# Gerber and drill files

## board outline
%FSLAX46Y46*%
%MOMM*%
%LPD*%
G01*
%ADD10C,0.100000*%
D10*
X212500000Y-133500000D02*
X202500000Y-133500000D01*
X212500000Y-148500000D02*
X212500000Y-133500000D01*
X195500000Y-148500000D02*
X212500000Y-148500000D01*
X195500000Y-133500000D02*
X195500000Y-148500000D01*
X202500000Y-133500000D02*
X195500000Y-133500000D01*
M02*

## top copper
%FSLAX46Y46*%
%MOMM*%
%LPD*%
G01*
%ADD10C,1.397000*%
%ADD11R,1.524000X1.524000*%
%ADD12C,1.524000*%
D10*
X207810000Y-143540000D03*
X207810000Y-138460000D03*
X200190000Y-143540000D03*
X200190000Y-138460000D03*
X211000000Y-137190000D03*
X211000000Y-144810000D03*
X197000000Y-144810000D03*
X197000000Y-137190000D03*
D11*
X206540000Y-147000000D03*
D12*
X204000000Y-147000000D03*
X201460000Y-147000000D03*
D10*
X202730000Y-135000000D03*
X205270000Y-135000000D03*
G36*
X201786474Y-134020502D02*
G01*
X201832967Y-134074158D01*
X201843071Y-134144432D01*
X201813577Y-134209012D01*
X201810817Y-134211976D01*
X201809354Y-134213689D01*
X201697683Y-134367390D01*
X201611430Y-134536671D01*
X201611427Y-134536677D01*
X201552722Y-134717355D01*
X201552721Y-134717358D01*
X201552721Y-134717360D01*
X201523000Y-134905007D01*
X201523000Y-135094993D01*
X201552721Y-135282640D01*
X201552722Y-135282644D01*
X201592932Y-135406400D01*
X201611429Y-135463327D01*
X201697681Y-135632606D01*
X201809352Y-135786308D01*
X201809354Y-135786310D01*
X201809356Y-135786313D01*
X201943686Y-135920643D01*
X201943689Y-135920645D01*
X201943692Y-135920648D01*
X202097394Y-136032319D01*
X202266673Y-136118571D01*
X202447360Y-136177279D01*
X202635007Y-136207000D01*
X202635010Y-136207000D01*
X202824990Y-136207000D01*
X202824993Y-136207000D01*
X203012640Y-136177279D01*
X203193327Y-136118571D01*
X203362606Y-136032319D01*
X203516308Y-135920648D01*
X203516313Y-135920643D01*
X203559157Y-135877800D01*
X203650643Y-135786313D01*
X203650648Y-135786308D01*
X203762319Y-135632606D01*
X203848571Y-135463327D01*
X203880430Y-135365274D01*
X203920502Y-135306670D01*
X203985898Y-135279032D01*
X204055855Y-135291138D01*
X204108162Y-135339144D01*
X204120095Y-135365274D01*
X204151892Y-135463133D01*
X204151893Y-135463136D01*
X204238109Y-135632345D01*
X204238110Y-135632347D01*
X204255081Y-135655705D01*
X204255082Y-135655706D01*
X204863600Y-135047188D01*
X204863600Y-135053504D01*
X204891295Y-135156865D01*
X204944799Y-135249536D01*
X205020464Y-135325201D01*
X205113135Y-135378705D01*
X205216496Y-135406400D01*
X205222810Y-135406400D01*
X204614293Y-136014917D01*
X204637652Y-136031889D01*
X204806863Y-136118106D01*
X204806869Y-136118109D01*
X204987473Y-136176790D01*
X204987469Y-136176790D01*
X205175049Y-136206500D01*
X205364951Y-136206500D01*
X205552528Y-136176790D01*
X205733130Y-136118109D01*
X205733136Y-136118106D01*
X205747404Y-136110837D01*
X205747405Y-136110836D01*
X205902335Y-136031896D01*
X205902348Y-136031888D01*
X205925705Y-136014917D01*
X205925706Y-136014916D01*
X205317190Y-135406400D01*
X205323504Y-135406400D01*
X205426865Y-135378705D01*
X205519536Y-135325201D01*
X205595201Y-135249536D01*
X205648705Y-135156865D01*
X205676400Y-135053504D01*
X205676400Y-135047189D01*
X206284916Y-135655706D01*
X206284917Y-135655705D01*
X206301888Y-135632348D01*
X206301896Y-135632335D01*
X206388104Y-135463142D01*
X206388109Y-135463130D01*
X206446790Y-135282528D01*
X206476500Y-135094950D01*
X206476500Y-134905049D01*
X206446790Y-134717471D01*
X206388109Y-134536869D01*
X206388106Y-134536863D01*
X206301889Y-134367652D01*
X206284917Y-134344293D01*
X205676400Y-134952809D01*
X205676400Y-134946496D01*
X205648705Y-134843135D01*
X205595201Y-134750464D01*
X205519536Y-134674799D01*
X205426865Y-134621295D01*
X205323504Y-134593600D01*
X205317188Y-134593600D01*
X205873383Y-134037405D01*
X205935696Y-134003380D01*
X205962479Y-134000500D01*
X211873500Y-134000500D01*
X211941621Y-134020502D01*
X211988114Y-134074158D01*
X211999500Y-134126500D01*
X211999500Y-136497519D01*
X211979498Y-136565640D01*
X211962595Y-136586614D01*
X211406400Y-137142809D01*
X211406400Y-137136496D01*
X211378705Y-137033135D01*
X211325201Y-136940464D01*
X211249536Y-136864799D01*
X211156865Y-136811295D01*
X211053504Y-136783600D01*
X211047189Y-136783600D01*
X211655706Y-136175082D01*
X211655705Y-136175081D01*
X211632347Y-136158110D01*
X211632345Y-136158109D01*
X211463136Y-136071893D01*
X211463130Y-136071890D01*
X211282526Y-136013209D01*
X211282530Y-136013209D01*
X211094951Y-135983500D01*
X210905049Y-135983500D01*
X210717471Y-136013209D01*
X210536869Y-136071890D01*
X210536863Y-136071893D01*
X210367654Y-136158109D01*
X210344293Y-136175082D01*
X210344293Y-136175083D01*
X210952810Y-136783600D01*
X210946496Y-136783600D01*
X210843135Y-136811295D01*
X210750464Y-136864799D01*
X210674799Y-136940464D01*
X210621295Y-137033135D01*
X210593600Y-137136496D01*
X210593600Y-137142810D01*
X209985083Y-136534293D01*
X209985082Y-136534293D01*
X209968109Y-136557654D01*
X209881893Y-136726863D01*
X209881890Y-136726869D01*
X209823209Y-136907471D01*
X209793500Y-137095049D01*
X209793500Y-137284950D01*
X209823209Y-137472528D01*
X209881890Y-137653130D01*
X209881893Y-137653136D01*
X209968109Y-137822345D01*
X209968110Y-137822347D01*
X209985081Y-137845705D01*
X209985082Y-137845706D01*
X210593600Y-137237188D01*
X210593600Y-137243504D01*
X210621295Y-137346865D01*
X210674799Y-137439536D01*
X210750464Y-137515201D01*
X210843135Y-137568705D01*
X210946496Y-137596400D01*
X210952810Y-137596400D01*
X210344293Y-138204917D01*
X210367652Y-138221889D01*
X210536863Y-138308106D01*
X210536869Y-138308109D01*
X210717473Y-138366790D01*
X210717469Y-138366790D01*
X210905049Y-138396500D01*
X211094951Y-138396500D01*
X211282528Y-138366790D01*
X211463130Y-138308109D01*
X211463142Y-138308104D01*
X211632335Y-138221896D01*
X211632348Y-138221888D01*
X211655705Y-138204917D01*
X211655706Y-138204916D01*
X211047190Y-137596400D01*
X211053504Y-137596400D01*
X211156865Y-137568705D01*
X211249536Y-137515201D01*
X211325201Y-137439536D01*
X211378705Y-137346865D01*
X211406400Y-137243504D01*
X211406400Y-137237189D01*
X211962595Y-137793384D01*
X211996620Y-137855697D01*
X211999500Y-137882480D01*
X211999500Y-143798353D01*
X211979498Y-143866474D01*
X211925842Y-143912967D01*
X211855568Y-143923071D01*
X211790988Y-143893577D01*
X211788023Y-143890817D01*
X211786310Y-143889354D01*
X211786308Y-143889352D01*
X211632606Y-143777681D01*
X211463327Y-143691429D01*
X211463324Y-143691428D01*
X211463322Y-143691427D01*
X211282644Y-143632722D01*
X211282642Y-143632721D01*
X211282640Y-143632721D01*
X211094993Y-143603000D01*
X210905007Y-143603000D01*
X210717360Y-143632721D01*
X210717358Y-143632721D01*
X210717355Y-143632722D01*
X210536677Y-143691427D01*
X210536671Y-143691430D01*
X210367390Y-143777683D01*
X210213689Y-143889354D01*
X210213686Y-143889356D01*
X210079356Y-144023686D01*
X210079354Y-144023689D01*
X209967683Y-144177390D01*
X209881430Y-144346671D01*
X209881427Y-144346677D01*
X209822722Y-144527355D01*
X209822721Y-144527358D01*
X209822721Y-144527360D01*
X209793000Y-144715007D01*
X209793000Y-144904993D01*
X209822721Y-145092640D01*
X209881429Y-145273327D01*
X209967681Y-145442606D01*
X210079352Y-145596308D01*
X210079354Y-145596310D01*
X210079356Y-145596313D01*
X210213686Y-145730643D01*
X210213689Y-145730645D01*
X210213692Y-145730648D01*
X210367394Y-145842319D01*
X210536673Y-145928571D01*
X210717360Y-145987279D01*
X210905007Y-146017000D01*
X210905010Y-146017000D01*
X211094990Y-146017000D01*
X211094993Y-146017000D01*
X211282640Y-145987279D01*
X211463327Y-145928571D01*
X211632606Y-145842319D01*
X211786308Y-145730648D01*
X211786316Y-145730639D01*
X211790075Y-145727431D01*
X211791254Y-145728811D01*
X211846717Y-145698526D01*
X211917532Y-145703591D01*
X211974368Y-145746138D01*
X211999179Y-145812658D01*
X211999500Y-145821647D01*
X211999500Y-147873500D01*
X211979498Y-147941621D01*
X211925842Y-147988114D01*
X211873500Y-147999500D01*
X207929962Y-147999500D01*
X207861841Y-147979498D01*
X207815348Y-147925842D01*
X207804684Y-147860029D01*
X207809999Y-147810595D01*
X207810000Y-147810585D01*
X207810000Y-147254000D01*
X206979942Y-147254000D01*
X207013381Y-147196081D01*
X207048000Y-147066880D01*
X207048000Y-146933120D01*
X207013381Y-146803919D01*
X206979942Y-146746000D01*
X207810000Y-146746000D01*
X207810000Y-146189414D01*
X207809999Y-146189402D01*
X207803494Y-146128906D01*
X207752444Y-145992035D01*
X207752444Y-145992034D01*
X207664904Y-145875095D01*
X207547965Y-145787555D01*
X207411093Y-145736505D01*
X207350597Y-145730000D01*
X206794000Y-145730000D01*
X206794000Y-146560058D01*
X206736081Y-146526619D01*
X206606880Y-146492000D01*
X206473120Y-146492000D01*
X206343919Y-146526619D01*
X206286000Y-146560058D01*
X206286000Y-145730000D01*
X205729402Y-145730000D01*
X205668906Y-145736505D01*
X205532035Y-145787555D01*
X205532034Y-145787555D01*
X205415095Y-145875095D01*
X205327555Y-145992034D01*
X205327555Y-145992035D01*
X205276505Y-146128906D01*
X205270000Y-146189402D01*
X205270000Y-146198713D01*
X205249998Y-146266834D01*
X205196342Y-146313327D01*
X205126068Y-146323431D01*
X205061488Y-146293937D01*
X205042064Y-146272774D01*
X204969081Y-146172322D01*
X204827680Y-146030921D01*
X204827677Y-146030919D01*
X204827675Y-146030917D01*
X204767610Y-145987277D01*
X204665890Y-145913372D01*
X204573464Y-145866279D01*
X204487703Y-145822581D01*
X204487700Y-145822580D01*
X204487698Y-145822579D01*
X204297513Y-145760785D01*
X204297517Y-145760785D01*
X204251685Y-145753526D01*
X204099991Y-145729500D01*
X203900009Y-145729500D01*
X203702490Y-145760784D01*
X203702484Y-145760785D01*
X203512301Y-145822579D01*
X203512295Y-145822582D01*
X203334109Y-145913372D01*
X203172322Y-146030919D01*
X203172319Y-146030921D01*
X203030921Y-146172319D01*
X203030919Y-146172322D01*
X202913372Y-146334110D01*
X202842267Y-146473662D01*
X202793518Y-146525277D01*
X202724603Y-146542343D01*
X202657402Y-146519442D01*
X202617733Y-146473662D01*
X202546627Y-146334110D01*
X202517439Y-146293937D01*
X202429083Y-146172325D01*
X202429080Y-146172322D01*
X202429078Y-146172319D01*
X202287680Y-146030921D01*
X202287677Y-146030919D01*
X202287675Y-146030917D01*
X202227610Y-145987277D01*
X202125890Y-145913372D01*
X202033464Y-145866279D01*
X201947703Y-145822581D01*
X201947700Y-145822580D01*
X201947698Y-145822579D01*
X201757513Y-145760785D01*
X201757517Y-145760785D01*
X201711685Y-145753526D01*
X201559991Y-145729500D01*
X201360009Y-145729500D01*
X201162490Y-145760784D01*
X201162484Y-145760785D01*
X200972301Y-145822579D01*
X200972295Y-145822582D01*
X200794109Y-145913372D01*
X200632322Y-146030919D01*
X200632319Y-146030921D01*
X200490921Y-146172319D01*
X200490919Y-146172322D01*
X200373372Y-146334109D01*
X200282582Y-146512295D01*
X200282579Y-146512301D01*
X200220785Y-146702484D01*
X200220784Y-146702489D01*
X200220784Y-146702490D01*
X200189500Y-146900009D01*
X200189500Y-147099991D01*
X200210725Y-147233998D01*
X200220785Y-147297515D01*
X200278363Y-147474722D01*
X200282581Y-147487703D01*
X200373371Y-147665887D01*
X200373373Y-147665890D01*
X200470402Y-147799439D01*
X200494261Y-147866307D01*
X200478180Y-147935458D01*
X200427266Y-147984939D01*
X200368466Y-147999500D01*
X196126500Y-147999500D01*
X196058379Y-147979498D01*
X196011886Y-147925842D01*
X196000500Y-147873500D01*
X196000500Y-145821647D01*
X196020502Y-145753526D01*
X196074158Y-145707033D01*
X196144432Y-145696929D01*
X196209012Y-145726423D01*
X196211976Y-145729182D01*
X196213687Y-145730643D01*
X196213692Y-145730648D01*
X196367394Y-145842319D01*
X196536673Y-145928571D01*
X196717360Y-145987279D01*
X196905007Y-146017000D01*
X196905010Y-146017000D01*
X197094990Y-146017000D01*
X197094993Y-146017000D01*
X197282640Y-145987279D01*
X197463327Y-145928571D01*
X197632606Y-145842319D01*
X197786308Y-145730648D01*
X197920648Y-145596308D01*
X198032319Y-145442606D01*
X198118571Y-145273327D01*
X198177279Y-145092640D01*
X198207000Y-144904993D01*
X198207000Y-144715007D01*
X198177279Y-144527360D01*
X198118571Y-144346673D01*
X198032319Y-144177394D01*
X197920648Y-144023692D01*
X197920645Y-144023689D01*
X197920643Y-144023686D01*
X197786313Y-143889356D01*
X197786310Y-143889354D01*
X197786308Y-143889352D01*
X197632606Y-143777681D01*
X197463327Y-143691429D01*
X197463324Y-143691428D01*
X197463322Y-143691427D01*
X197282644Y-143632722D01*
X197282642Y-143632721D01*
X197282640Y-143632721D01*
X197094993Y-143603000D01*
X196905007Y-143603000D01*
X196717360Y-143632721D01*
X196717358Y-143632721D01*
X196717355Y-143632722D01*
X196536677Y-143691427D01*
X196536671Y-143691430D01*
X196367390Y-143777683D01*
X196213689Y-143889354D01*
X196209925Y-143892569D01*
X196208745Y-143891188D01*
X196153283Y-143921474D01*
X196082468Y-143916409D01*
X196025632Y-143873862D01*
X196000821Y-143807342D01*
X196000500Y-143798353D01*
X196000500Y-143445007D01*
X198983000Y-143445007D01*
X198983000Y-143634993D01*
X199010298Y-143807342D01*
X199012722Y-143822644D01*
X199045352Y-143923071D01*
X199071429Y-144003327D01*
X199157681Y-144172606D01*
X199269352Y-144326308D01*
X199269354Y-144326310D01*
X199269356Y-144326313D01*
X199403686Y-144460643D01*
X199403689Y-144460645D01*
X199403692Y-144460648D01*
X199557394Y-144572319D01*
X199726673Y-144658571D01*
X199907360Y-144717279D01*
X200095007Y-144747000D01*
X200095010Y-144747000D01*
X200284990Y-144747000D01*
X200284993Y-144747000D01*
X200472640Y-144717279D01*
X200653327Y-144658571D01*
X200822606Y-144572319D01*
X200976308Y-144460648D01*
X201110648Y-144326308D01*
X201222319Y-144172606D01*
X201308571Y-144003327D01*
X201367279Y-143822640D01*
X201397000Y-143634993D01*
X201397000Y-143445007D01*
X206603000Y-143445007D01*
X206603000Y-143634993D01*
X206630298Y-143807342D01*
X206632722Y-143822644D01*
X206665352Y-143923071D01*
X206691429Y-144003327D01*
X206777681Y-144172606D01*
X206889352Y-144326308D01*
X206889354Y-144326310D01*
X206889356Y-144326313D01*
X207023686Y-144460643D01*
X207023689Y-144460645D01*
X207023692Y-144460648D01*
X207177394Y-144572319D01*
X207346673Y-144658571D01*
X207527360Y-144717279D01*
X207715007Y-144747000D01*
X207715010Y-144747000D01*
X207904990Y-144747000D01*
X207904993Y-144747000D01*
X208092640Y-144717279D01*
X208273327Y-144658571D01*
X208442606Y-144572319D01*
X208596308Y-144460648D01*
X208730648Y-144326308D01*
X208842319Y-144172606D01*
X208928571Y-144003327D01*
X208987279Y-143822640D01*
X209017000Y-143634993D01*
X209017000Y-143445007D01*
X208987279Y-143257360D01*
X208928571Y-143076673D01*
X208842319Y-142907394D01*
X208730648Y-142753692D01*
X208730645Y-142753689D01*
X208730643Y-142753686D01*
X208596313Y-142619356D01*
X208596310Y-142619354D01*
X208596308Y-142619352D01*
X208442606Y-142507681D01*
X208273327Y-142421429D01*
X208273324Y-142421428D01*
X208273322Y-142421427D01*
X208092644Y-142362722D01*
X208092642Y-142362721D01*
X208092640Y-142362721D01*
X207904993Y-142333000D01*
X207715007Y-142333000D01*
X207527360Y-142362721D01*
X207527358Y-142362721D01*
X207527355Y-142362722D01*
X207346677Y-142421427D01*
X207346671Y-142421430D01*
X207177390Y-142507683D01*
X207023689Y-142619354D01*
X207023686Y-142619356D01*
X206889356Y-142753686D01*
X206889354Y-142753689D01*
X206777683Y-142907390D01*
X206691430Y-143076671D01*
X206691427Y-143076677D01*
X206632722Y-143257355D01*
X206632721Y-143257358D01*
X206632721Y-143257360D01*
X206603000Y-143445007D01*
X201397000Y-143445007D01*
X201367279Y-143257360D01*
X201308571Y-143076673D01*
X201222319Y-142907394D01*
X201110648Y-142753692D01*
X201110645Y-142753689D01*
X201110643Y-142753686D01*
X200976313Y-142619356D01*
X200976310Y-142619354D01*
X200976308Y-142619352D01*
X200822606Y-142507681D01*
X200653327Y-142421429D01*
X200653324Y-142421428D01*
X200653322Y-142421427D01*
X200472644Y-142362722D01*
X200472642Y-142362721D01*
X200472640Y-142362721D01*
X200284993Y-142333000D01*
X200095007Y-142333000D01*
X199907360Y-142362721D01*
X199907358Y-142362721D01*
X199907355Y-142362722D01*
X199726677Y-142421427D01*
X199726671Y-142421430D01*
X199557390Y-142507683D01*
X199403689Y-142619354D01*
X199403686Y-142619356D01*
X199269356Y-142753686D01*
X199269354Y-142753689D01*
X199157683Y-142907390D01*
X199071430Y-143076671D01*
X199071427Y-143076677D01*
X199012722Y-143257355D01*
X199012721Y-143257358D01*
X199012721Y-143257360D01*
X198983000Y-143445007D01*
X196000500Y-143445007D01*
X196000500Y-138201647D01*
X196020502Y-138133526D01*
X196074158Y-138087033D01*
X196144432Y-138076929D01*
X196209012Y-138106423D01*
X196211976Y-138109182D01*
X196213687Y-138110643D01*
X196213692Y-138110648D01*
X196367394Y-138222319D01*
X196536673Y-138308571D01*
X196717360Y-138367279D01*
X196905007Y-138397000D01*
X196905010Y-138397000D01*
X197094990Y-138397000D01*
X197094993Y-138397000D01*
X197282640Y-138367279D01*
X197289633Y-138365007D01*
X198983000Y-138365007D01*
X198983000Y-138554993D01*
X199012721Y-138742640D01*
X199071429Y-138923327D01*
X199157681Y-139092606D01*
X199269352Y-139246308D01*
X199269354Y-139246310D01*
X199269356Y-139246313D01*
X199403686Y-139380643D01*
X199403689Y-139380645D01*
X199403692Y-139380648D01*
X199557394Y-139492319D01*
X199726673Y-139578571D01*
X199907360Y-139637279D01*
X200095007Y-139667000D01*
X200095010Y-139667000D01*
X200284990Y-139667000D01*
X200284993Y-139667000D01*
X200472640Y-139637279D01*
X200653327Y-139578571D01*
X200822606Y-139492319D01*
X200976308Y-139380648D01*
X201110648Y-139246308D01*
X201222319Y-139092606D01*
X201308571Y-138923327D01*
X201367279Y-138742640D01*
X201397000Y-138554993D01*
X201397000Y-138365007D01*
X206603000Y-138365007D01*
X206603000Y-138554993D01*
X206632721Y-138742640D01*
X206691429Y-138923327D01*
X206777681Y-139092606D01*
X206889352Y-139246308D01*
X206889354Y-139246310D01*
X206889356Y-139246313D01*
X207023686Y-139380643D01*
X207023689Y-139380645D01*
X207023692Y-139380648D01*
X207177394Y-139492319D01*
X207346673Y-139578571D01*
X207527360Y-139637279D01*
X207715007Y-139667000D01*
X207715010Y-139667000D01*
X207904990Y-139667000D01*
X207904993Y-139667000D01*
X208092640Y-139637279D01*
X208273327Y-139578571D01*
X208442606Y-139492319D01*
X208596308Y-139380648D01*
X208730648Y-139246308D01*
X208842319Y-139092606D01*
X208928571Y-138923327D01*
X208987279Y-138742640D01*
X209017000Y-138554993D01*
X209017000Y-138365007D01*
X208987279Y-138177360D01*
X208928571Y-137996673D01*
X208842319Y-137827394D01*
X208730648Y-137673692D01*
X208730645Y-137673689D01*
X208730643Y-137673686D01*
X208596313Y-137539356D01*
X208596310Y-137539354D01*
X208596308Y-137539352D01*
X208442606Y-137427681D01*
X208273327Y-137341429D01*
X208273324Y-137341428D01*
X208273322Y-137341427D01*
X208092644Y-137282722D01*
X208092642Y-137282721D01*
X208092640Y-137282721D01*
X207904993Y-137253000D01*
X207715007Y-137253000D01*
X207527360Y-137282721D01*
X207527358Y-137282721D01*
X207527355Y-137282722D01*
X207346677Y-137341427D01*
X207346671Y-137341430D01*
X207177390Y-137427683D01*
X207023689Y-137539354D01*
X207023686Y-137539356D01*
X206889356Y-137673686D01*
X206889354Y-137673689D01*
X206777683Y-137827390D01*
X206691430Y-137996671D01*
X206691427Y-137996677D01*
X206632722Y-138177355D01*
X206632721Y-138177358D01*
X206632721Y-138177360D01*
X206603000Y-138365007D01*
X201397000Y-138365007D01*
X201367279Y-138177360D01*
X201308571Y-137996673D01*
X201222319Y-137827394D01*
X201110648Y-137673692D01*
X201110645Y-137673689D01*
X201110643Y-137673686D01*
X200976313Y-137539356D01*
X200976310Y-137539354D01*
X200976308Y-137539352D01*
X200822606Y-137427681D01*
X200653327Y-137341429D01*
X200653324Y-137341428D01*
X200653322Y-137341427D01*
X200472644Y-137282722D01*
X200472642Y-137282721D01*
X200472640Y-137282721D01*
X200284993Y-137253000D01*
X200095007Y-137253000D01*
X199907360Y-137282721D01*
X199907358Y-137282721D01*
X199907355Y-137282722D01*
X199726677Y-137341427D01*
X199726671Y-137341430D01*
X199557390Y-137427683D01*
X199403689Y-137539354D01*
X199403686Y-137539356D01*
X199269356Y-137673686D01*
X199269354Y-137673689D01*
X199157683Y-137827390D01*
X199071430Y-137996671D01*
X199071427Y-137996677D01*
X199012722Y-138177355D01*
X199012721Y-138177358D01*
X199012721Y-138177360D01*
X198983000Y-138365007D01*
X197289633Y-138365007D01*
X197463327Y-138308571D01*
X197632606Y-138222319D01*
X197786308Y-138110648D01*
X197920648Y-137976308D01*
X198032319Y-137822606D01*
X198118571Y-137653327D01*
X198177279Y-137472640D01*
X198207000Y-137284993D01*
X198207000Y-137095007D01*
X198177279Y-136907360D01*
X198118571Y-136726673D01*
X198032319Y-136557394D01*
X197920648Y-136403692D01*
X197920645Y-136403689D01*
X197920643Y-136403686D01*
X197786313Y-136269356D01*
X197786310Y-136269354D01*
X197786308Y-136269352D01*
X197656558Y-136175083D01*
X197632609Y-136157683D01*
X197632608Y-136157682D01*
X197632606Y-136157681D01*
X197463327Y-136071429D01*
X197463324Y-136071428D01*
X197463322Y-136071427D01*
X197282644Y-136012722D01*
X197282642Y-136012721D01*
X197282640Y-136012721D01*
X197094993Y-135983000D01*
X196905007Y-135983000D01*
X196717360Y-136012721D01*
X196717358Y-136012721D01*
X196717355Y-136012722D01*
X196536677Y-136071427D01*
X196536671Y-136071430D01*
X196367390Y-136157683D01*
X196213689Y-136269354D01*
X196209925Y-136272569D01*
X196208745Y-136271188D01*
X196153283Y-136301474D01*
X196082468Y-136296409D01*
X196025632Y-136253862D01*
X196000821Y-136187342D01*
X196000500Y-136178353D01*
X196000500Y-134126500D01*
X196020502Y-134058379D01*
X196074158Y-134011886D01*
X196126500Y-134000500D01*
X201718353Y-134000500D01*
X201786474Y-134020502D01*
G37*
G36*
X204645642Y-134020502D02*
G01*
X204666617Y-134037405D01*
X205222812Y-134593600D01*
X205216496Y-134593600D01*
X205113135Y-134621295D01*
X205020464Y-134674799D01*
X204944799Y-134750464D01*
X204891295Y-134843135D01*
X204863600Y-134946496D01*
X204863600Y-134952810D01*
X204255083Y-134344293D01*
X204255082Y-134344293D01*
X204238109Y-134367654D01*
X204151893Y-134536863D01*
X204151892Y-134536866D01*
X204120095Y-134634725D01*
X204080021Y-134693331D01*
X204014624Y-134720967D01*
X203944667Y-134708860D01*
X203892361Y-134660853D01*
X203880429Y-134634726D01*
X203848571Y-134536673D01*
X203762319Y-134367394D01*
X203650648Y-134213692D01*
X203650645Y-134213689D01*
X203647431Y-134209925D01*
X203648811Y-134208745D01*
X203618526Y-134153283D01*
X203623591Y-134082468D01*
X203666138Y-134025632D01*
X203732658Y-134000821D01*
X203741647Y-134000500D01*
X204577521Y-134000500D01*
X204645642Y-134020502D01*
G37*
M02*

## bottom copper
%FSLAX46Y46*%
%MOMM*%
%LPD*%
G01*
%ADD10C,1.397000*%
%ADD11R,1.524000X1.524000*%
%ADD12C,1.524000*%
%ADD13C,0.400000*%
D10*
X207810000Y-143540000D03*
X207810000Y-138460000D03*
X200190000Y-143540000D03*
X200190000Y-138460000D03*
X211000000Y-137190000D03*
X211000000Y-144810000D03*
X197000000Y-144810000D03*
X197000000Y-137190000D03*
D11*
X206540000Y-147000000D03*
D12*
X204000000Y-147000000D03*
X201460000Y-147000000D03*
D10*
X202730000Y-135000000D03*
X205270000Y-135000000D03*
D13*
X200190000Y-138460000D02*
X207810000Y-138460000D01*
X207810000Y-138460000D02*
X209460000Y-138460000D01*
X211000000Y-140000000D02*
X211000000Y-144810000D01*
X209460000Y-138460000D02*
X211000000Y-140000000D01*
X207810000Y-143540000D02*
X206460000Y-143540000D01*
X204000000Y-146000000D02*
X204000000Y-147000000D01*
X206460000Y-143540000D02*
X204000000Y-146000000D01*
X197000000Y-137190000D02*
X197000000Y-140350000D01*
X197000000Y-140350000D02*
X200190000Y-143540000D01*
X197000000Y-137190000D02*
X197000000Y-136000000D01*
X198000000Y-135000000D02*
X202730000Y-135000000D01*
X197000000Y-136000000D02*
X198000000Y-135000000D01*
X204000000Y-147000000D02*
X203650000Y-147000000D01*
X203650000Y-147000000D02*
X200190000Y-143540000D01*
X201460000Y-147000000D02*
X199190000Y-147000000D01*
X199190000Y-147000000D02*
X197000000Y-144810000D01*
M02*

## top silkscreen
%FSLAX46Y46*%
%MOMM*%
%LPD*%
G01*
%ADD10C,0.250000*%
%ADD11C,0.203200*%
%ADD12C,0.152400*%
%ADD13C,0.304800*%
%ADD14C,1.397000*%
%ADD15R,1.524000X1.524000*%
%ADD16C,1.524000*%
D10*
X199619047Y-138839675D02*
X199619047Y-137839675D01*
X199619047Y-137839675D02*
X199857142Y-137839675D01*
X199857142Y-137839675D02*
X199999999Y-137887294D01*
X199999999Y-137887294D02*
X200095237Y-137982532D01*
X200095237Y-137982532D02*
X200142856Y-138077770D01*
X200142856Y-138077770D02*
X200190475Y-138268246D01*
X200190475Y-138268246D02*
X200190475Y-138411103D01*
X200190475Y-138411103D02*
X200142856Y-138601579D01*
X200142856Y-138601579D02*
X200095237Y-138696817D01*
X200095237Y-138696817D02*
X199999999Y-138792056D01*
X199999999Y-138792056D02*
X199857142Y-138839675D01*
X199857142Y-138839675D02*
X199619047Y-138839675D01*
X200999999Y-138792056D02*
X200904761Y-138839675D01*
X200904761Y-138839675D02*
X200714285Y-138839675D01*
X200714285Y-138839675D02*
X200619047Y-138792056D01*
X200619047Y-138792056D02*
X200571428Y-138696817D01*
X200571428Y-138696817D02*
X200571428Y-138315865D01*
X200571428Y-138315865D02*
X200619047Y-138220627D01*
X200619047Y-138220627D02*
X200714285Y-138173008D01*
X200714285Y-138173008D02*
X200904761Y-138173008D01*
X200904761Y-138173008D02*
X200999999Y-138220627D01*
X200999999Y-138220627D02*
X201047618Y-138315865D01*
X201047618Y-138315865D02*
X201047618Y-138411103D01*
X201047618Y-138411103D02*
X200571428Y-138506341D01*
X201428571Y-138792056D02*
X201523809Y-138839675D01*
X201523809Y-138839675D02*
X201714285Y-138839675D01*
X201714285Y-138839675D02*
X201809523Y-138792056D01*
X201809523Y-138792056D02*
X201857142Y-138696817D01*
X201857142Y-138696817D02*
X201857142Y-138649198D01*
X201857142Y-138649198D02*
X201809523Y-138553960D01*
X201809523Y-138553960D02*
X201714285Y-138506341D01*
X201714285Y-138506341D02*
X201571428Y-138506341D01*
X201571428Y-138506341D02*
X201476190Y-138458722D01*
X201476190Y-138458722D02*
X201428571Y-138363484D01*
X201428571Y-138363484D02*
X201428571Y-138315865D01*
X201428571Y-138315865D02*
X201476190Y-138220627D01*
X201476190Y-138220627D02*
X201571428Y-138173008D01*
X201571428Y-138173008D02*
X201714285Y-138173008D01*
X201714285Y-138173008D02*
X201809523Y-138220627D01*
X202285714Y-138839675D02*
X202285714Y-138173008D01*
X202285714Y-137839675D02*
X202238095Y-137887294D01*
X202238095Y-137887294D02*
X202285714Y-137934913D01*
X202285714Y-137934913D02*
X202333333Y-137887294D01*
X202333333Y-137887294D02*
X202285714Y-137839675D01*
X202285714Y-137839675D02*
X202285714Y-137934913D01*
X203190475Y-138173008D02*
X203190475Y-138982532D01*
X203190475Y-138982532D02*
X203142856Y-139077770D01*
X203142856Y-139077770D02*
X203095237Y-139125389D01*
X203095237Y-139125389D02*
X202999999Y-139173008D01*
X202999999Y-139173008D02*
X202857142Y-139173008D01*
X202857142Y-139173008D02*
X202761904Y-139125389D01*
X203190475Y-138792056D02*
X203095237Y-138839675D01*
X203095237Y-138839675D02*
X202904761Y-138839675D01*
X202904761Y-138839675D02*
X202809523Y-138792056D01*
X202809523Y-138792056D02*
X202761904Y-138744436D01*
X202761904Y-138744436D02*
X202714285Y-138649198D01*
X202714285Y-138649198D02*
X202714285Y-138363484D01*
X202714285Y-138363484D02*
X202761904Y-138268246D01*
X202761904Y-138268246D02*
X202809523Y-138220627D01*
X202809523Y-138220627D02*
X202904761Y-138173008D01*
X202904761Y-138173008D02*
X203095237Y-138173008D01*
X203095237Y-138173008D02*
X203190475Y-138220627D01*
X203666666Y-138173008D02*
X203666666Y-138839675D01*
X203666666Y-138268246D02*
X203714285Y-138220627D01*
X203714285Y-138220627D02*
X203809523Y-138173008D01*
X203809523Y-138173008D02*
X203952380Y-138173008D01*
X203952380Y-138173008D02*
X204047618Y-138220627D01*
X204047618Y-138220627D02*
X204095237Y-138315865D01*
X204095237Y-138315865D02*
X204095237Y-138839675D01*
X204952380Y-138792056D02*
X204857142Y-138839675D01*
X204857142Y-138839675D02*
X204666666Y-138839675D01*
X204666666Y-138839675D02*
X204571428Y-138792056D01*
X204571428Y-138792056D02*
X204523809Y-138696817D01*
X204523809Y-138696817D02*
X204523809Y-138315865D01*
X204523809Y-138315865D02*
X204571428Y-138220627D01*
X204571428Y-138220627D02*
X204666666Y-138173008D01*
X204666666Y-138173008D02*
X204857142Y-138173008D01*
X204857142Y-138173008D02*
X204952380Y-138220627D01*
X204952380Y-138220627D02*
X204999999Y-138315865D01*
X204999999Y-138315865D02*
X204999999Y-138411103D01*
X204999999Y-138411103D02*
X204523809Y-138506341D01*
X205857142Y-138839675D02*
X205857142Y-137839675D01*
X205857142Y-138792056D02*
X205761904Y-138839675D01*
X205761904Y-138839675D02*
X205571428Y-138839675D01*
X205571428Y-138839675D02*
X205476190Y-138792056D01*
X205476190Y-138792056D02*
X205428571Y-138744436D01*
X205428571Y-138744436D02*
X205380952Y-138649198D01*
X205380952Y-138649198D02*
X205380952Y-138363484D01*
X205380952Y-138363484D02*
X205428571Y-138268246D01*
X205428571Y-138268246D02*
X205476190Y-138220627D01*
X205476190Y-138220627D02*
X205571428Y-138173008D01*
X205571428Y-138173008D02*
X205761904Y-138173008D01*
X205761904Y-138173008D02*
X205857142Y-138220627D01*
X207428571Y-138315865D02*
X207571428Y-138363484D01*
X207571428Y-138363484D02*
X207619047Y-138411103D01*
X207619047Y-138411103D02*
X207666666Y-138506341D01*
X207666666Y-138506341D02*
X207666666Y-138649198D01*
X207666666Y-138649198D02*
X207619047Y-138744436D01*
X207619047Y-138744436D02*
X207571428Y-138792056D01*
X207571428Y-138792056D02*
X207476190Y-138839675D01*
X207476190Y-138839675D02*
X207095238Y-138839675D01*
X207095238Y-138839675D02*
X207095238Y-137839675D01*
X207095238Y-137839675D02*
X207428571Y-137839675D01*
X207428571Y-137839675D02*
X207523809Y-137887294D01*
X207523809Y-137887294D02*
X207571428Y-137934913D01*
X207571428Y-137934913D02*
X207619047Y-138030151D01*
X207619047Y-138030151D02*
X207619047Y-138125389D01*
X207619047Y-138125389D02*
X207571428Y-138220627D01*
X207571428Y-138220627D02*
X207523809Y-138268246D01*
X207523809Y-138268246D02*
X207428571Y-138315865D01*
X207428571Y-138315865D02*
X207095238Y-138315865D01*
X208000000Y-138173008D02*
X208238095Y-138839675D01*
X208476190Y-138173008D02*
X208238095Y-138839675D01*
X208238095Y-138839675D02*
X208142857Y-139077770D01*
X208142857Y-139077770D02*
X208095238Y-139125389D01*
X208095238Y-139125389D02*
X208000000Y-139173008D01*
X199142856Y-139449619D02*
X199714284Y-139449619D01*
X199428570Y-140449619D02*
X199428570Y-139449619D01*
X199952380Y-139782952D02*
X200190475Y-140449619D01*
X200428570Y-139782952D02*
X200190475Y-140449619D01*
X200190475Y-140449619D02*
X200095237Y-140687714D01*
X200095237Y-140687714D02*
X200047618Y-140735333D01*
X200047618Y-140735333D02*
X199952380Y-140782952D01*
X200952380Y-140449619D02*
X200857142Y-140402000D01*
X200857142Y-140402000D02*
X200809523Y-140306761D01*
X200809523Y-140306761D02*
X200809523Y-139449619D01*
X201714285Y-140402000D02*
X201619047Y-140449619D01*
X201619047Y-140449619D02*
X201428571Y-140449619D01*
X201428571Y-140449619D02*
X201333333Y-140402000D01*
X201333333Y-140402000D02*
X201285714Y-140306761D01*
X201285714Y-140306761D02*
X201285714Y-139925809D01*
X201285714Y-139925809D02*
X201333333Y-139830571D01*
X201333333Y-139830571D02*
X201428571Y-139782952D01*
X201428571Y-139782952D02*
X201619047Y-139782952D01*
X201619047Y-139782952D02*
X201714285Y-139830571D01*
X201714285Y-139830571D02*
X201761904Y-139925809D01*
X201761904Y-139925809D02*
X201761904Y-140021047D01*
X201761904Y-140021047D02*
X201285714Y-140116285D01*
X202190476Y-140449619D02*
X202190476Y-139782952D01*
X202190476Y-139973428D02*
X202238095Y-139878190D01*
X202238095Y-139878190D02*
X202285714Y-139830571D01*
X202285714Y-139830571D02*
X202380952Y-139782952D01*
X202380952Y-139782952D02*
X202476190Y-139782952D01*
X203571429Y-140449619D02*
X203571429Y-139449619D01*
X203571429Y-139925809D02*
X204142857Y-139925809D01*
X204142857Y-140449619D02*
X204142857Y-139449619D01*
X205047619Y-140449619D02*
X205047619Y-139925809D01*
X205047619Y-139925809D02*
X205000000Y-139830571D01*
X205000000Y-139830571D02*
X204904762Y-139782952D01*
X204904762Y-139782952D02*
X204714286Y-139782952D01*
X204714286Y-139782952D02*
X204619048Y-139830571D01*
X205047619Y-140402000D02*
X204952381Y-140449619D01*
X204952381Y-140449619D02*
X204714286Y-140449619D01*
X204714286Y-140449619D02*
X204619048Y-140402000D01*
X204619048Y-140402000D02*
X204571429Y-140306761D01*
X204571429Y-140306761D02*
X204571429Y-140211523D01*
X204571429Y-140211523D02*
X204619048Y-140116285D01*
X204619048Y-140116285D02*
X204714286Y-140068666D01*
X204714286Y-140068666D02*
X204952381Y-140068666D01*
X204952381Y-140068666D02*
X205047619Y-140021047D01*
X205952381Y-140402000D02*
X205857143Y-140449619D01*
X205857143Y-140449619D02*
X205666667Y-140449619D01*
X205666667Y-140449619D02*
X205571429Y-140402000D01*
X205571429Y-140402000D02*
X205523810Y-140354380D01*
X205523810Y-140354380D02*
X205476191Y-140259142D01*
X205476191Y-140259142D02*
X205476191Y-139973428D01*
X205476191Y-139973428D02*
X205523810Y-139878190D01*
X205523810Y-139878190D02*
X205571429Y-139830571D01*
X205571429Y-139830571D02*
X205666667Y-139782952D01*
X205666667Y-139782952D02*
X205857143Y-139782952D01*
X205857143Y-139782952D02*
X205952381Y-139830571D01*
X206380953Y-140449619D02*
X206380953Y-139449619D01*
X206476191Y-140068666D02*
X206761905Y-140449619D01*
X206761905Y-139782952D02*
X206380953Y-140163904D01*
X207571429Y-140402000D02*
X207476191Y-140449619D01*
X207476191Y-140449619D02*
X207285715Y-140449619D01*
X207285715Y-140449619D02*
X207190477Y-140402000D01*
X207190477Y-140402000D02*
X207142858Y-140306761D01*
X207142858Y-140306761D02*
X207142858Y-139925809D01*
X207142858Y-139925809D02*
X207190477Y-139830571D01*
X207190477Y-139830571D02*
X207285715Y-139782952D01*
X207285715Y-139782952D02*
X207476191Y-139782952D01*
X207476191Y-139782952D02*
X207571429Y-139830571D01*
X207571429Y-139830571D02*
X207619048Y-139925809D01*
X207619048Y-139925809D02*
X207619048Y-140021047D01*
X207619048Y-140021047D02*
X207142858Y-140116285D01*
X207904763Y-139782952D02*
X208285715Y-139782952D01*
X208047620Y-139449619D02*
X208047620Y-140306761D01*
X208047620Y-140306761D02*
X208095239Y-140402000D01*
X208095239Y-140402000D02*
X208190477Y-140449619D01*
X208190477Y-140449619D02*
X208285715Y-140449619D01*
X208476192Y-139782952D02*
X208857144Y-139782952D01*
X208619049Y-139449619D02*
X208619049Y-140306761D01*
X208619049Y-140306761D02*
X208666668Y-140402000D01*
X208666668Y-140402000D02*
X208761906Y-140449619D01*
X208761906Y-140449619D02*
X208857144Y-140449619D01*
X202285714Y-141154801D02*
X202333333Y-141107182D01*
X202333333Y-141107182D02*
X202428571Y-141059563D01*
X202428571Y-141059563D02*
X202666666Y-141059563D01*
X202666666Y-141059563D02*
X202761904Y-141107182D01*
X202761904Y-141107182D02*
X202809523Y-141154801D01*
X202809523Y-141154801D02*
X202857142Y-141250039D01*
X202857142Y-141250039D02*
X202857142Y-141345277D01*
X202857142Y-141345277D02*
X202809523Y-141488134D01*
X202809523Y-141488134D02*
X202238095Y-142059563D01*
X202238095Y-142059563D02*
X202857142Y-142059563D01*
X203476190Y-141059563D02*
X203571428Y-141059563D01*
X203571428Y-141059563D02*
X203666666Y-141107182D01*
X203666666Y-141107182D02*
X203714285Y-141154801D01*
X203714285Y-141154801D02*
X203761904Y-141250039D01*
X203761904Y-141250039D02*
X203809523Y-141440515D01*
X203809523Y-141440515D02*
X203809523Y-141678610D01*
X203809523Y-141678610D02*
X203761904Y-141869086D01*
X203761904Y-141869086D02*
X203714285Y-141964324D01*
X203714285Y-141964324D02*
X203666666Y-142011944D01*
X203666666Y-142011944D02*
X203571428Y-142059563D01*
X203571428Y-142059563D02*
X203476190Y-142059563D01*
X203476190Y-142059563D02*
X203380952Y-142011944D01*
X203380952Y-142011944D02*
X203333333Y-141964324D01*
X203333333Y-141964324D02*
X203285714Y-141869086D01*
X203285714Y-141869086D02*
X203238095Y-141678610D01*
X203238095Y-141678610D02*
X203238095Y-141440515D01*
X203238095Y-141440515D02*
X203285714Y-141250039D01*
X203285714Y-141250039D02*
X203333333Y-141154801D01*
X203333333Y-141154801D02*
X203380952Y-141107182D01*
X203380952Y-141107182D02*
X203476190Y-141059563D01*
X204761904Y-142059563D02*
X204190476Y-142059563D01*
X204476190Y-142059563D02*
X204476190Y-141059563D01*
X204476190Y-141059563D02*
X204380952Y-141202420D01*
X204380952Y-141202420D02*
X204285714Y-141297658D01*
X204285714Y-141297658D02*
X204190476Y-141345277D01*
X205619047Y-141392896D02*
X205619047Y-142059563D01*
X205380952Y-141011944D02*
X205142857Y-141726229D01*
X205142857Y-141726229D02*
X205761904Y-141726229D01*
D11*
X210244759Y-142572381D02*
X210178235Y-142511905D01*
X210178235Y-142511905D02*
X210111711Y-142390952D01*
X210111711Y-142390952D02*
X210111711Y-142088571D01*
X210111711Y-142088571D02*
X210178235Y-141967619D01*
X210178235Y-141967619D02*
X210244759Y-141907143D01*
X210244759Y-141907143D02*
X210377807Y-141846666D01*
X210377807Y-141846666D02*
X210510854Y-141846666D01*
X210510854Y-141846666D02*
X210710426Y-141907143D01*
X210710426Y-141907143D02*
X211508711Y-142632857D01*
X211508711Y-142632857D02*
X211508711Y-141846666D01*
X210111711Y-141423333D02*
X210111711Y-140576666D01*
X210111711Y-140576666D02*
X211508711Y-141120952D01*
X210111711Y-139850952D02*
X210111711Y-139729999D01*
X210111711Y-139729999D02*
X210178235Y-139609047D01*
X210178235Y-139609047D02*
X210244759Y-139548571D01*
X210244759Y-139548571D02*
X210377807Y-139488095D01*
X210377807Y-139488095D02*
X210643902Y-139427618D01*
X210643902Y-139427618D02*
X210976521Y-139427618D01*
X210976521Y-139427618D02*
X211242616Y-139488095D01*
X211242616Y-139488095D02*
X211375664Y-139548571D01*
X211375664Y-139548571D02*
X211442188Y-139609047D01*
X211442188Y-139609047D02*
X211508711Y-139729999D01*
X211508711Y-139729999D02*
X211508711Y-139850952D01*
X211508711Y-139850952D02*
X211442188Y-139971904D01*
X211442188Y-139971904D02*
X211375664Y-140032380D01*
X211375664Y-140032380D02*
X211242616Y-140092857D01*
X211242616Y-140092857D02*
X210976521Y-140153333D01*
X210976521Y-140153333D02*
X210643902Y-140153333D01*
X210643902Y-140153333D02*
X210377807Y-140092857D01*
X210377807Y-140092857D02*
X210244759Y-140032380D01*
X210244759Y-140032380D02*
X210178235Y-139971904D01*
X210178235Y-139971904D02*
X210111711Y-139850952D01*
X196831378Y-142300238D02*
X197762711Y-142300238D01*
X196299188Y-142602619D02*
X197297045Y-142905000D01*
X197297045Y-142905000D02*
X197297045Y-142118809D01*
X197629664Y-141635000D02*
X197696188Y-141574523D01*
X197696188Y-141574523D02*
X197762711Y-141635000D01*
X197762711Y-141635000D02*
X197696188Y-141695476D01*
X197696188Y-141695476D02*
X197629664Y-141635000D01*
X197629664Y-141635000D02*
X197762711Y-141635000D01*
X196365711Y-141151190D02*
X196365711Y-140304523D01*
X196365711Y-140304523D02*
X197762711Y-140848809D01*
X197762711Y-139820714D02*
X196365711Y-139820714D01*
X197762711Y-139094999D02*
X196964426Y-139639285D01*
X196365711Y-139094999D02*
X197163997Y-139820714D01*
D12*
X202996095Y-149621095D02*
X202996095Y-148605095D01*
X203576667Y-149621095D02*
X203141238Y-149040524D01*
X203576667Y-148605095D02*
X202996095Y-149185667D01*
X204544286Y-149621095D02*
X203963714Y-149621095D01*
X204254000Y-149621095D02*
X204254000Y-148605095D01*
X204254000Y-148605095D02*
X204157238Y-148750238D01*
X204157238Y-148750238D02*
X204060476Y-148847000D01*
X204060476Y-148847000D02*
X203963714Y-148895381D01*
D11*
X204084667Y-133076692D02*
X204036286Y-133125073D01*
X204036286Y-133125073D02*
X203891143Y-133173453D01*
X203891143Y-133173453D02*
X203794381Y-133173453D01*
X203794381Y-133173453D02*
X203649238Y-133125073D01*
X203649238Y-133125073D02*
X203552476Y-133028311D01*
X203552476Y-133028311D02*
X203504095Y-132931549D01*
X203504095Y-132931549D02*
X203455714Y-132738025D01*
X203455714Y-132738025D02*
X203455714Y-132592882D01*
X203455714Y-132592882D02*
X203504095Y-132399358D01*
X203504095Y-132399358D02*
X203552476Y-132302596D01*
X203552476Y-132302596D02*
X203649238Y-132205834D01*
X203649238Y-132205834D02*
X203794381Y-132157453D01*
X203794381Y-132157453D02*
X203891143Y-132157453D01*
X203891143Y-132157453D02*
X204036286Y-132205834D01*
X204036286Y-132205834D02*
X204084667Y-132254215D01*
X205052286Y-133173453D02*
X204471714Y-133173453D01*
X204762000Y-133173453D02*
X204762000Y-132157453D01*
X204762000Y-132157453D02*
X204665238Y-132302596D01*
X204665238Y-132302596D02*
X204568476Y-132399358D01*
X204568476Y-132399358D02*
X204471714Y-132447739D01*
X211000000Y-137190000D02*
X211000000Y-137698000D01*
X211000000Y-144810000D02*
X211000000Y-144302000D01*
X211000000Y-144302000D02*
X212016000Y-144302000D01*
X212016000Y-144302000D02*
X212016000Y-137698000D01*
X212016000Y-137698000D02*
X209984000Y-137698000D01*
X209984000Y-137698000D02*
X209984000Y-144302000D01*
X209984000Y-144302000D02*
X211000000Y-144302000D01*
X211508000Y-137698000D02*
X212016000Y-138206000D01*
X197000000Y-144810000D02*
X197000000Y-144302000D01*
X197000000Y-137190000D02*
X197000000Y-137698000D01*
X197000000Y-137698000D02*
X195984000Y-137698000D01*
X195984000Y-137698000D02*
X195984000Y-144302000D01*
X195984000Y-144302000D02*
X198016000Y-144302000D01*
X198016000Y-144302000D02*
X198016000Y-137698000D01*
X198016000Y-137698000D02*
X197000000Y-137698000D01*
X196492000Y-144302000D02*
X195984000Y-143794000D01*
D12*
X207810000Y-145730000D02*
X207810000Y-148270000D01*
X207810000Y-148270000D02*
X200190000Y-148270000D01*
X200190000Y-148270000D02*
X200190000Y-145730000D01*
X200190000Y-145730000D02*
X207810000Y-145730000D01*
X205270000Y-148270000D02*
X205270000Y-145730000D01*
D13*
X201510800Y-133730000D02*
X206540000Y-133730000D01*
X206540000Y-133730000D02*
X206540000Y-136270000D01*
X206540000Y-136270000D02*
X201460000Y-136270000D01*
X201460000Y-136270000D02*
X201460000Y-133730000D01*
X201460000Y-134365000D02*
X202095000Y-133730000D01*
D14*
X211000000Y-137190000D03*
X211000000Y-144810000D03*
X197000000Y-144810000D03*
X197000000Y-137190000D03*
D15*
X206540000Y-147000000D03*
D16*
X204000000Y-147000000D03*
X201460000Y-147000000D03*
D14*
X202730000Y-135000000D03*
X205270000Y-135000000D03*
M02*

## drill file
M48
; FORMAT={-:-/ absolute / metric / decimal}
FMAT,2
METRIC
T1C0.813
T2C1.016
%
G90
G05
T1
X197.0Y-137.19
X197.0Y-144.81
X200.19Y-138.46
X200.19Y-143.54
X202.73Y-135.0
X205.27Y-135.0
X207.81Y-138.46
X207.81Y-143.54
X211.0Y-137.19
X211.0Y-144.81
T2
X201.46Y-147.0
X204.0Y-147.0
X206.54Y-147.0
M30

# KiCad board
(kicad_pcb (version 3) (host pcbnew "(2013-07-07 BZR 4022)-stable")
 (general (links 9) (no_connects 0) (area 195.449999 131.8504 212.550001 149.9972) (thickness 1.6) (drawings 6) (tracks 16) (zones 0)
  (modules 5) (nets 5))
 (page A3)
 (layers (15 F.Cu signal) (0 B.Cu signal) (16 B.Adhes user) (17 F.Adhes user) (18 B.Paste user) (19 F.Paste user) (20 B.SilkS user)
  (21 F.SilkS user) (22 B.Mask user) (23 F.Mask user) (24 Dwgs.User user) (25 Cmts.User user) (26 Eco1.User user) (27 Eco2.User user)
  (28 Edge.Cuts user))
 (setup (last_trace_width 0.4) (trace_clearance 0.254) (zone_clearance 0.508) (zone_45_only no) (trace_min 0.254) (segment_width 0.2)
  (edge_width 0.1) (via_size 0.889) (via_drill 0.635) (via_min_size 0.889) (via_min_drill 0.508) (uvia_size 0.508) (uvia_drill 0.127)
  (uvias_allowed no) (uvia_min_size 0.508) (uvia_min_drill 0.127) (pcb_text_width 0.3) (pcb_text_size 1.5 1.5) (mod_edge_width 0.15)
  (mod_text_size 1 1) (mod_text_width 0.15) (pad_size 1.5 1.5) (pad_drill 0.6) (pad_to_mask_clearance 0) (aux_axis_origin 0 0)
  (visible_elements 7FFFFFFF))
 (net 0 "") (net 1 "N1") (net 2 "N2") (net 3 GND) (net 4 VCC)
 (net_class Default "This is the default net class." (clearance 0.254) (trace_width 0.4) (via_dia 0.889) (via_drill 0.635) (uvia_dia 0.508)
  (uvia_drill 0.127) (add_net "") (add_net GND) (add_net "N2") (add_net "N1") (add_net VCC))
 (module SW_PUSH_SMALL (layer B.Cu) (at 204 141)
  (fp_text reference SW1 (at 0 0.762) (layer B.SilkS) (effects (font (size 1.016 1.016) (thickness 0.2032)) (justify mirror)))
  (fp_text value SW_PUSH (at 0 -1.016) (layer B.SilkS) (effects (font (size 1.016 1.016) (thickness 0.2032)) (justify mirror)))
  (pad 1 thru_hole circle (at 3.81 2.54) (size 1.397 1.397) (drill 0.8128) (layers *.Cu *.Mask B.SilkS) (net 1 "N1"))
  (pad 2 thru_hole circle (at 3.81 -2.54) (size 1.397 1.397) (drill 0.8128) (layers *.Cu *.Mask B.SilkS) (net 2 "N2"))
  (pad 1 thru_hole circle (at -3.81 2.54) (size 1.397 1.397) (drill 0.8128) (layers *.Cu *.Mask B.SilkS) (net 1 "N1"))
  (pad 2 thru_hole circle (at -3.81 -2.54) (size 1.397 1.397) (drill 0.8128) (layers *.Cu *.Mask B.SilkS) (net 2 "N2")))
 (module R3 (layer F.Cu) (at 211 141 270) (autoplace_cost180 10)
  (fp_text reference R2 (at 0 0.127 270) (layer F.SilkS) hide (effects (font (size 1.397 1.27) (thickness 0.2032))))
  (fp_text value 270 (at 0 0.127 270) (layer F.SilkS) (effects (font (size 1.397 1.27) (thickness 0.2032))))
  (fp_line (start -3.81 0) (end -3.302 0) (layer F.SilkS) (width 0.2032))
  (fp_line (start 3.81 0) (end 3.302 0) (layer F.SilkS) (width 0.2032))
  (fp_line (start 3.302 0) (end 3.302 -1.016) (layer F.SilkS) (width 0.2032))
  (fp_line (start 3.302 -1.016) (end -3.302 -1.016) (layer F.SilkS) (width 0.2032))
  (fp_line (start -3.302 -1.016) (end -3.302 1.016) (layer F.SilkS) (width 0.2032))
  (fp_line (start -3.302 1.016) (end 3.302 1.016) (layer F.SilkS) (width 0.2032))
  (fp_line (start 3.302 1.016) (end 3.302 0) (layer F.SilkS) (width 0.2032))
  (fp_line (start -3.302 -0.508) (end -2.794 -1.016) (layer F.SilkS) (width 0.2032))
  (pad 1 thru_hole circle (at -3.81 0 270) (size 1.397 1.397) (drill 0.8128) (layers *.Cu *.Mask F.SilkS) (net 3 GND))
  (pad 2 thru_hole circle (at 3.81 0 270) (size 1.397 1.397) (drill 0.8128) (layers *.Cu *.Mask F.SilkS) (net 2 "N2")))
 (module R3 (layer F.Cu) (at 197 141 90) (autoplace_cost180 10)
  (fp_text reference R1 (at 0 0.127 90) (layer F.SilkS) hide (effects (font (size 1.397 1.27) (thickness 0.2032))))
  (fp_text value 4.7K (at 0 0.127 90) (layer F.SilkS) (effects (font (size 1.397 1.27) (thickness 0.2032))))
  (fp_line (start -3.81 0) (end -3.302 0) (layer F.SilkS) (width 0.2032))
  (fp_line (start 3.81 0) (end 3.302 0) (layer F.SilkS) (width 0.2032))
  (fp_line (start 3.302 0) (end 3.302 -1.016) (layer F.SilkS) (width 0.2032))
  (fp_line (start 3.302 -1.016) (end -3.302 -1.016) (layer F.SilkS) (width 0.2032))
  (fp_line (start -3.302 -1.016) (end -3.302 1.016) (layer F.SilkS) (width 0.2032))
  (fp_line (start -3.302 1.016) (end 3.302 1.016) (layer F.SilkS) (width 0.2032))
  (fp_line (start 3.302 1.016) (end 3.302 0) (layer F.SilkS) (width 0.2032))
  (fp_line (start -3.302 -0.508) (end -2.794 -1.016) (layer F.SilkS) (width 0.2032))
  (pad 1 thru_hole circle (at -3.81 0 90) (size 1.397 1.397) (drill 0.8128) (layers *.Cu *.Mask F.SilkS) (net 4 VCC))
  (pad 2 thru_hole circle (at 3.81 0 90) (size 1.397 1.397) (drill 0.8128) (layers *.Cu *.Mask F.SilkS) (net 1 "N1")))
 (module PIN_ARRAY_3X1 (layer F.Cu) (at 204 147 180)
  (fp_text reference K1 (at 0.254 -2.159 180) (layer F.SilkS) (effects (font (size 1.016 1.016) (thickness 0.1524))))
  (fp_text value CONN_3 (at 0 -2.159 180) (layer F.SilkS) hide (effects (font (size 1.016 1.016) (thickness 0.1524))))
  (fp_line (start -3.81 1.27) (end -3.81 -1.27) (layer F.SilkS) (width 0.1524))
  (fp_line (start -3.81 -1.27) (end 3.81 -1.27) (layer F.SilkS) (width 0.1524))
  (fp_line (start 3.81 -1.27) (end 3.81 1.27) (layer F.SilkS) (width 0.1524))
  (fp_line (start 3.81 1.27) (end -3.81 1.27) (layer F.SilkS) (width 0.1524))
  (fp_line (start -1.27 -1.27) (end -1.27 1.27) (layer F.SilkS) (width 0.1524))
  (pad 1 thru_hole rect (at -2.54 0 180) (size 1.524 1.524) (drill 1.016) (layers *.Cu *.Mask F.SilkS) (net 3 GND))
  (pad 2 thru_hole circle (at 0 0 180) (size 1.524 1.524) (drill 1.016) (layers *.Cu *.Mask F.SilkS) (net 1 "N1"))
  (pad 3 thru_hole circle (at 2.54 0 180) (size 1.524 1.524) (drill 1.016) (layers *.Cu *.Mask F.SilkS) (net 4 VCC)))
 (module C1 (layer F.Cu) (at 204 135)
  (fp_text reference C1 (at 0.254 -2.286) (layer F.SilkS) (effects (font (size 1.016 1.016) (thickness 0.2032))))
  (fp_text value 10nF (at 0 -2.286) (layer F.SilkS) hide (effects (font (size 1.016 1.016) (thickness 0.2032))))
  (fp_line (start -2.4892 -1.27) (end 2.54 -1.27) (layer F.SilkS) (width 0.3048))
  (fp_line (start 2.54 -1.27) (end 2.54 1.27) (layer F.SilkS) (width 0.3048))
  (fp_line (start 2.54 1.27) (end -2.54 1.27) (layer F.SilkS) (width 0.3048))
  (fp_line (start -2.54 1.27) (end -2.54 -1.27) (layer F.SilkS) (width 0.3048))
  (fp_line (start -2.54 -0.635) (end -1.905 -1.27) (layer F.SilkS) (width 0.3048))
  (pad 1 thru_hole circle (at -1.27 0) (size 1.397 1.397) (drill 0.8128) (layers *.Cu *.Mask F.SilkS) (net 1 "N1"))
  (pad 2 thru_hole circle (at 1.27 0) (size 1.397 1.397) (drill 0.8128) (layers *.Cu *.Mask F.SilkS) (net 3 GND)))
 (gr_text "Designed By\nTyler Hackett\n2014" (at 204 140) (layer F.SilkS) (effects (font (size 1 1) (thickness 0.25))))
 (gr_line (start 212.5 133.5) (end 202.5 133.5) (angle 90) (layer Edge.Cuts) (width 0.1))
 (gr_line (start 212.5 148.5) (end 212.5 133.5) (angle 90) (layer Edge.Cuts) (width 0.1))
 (gr_line (start 195.5 148.5) (end 212.5 148.5) (angle 90) (layer Edge.Cuts) (width 0.1))
 (gr_line (start 195.5 133.5) (end 195.5 148.5) (angle 90) (layer Edge.Cuts) (width 0.1))
 (gr_line (start 202.5 133.5) (end 195.5 133.5) (angle 90) (layer Edge.Cuts) (width 0.1))
 (segment (start 200.19 138.46) (end 207.81 138.46) (width 0.4) (layer B.Cu) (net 2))
 (segment (start 207.81 138.46) (end 209.46 138.46) (width 0.4) (layer B.Cu) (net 2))
 (segment (start 211 140) (end 211 144.81) (width 0.4) (layer B.Cu) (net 2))
 (segment (start 209.46 138.46) (end 211 140) (width 0.4) (layer B.Cu) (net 2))
 (segment (start 207.81 143.54) (end 206.46 143.54) (width 0.4) (layer B.Cu) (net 1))
 (segment (start 204 146) (end 204 147) (width 0.4) (layer B.Cu) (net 1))
 (segment (start 206.46 143.54) (end 204 146) (width 0.4) (layer B.Cu) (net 1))
 (segment (start 197 137.19) (end 197 140.35) (width 0.4) (layer B.Cu) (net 1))
 (segment (start 197 140.35) (end 200.19 143.54) (width 0.4) (layer B.Cu) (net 1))
 (segment (start 197 137.19) (end 197 136) (width 0.4) (layer B.Cu) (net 1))
 (segment (start 198 135) (end 202.73 135) (width 0.4) (layer B.Cu) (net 1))
 (segment (start 197 136) (end 198 135) (width 0.4) (layer B.Cu) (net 1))
 (segment (start 204 147) (end 203.65 147) (width 0.4) (layer B.Cu) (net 1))
 (segment (start 203.65 147) (end 200.19 143.54) (width 0.4) (layer B.Cu) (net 1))
 (segment (start 201.46 147) (end 199.19 147) (width 0.4) (layer B.Cu) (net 4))
 (segment (start 199.19 147) (end 197 144.81) (width 0.4) (layer B.Cu) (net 4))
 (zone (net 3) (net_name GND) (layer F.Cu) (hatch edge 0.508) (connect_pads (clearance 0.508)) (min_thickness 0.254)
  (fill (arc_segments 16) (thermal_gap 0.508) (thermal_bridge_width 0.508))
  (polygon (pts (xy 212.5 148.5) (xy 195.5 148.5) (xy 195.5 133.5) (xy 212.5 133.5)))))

